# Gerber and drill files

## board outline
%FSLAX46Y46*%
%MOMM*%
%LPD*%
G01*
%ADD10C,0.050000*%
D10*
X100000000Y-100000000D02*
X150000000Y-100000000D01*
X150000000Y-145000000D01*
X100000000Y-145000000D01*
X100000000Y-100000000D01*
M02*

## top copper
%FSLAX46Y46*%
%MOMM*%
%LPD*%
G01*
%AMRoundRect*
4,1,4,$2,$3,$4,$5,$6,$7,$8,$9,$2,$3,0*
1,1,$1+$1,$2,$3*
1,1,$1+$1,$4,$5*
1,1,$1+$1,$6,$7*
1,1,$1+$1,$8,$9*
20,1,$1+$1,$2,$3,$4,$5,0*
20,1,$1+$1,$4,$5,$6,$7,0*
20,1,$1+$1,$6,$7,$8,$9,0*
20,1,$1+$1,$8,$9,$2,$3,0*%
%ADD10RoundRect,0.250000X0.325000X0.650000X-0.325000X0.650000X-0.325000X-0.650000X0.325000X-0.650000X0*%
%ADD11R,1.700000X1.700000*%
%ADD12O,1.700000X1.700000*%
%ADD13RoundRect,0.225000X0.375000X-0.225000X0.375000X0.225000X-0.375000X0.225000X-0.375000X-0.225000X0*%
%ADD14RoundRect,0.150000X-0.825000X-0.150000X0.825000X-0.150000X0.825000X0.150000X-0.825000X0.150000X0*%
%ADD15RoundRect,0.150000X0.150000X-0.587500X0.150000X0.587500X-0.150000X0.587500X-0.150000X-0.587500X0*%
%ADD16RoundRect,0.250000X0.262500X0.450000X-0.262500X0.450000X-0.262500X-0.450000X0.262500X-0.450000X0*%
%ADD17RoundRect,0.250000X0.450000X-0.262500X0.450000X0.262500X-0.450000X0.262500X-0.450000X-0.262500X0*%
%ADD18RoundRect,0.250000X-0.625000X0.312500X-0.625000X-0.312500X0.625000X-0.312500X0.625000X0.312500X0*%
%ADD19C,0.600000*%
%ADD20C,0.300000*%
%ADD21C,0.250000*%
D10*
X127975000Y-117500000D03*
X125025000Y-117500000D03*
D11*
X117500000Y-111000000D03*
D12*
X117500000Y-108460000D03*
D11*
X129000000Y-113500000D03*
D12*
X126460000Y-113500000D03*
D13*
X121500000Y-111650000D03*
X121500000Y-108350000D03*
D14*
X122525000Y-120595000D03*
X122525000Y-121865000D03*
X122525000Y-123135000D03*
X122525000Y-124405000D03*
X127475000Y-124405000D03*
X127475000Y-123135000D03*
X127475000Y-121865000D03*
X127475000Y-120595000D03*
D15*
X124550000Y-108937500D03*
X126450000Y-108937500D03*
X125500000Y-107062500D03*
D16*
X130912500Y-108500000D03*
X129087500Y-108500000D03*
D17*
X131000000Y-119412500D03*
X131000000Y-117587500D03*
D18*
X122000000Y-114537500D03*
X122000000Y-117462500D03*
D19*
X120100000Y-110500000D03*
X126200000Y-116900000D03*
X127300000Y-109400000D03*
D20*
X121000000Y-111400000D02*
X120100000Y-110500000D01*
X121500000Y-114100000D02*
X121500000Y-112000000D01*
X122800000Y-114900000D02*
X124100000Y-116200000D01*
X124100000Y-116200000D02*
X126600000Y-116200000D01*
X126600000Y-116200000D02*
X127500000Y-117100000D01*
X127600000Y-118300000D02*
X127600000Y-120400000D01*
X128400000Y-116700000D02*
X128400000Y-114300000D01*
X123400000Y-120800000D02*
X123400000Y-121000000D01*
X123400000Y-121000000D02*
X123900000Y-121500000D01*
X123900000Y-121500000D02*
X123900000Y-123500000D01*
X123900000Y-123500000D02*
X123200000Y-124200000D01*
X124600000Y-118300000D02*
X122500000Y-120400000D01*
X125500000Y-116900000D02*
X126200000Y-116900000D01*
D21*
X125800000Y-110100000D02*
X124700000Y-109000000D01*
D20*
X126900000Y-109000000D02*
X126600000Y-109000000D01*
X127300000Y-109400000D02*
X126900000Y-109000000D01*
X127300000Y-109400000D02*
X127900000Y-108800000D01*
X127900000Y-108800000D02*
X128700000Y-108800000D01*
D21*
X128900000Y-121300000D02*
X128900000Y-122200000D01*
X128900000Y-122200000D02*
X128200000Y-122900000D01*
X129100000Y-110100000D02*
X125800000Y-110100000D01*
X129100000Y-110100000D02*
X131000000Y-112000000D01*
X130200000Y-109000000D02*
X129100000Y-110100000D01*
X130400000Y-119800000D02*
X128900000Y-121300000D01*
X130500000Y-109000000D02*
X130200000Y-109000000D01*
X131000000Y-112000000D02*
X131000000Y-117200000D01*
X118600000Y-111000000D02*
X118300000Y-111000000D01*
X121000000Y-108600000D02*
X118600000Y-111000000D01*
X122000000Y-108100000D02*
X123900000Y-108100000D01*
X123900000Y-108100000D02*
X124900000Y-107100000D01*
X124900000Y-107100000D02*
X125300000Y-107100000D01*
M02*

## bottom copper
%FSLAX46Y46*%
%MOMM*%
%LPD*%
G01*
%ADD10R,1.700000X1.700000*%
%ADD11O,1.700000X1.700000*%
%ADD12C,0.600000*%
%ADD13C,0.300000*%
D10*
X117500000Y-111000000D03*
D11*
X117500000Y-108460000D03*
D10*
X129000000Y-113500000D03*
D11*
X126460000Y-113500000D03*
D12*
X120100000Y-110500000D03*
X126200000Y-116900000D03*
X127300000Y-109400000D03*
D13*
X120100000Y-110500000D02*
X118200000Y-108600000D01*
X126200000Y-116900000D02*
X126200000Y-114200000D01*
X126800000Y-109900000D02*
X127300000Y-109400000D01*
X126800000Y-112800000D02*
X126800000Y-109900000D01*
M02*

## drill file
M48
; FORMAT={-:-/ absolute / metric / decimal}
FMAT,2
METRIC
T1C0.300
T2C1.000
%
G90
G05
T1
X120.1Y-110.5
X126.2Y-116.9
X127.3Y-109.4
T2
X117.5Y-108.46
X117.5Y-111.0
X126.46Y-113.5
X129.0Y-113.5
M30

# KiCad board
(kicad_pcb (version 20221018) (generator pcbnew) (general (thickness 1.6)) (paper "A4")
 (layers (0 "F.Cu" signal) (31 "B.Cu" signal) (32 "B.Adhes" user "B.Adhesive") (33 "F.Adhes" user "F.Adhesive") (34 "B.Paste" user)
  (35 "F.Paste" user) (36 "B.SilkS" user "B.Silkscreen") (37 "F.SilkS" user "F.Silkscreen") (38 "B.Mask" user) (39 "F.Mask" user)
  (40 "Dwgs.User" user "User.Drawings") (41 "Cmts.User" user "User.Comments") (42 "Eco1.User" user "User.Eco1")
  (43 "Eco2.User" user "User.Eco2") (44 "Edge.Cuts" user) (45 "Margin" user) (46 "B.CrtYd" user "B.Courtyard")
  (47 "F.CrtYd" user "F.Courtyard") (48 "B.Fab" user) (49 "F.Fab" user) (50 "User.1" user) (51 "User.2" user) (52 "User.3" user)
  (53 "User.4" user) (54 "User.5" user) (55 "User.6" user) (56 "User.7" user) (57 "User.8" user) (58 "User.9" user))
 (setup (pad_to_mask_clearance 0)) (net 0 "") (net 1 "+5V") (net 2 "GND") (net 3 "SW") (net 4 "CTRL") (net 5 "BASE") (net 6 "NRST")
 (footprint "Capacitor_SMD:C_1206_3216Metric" (layer "F.Cu") (at 126.5 117.5 180)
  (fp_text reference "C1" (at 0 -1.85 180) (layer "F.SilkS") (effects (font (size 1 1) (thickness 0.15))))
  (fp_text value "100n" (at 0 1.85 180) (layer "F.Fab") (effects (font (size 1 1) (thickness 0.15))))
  (pad "1" smd roundrect (at -1.475 0 180) (size 1.15 1.8) (layers "F.Cu" "F.Paste" "F.Mask") (roundrect_rratio 0.217391) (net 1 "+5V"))
  (pad "2" smd roundrect (at 1.475 0 180) (size 1.15 1.8) (layers "F.Cu" "F.Paste" "F.Mask") (roundrect_rratio 0.217391) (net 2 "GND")))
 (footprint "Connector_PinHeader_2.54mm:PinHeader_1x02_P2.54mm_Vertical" (layer "F.Cu") (at 117.5 111 180)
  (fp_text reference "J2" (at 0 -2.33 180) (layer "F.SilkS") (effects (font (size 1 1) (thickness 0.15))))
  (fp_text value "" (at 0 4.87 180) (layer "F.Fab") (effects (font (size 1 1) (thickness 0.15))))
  (pad "1" thru_hole rect (at 0 0 180) (size 1.7 1.7) (drill 1) (layers "*.Cu" "*.Mask") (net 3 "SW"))
  (pad "2" thru_hole oval (at 0 2.54 180) (size 1.7 1.7) (drill 1) (layers "*.Cu" "*.Mask") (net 1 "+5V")))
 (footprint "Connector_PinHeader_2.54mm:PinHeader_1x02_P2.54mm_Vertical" (layer "F.Cu") (at 129 113.5 -90)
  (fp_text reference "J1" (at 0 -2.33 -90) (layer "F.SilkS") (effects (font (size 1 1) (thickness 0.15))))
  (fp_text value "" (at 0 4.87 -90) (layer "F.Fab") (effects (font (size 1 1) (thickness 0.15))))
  (pad "1" thru_hole rect (at 0 0 270) (size 1.7 1.7) (drill 1) (layers "*.Cu" "*.Mask") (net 1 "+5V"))
  (pad "2" thru_hole oval (at 0 2.54 270) (size 1.7 1.7) (drill 1) (layers "*.Cu" "*.Mask") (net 2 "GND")))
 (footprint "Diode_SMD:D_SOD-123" (layer "F.Cu") (at 121.5 110 90)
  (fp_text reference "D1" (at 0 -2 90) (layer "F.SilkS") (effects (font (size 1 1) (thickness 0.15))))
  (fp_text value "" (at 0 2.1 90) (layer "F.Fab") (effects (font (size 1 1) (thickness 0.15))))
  (pad "1" smd roundrect (at -1.65 0 90) (size 0.9 1.2) (layers "F.Cu" "F.Paste" "F.Mask") (roundrect_rratio 0.25) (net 1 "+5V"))
  (pad "2" smd roundrect (at 1.65 0 90) (size 0.9 1.2) (layers "F.Cu" "F.Paste" "F.Mask") (roundrect_rratio 0.25) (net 3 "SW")))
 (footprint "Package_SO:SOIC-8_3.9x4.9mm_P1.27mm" (layer "F.Cu") (at 125 122.5)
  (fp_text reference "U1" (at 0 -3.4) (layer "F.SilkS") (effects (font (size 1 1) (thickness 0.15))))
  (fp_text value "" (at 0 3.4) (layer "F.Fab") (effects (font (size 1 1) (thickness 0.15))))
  (pad "1" smd roundrect (at -2.475 -1.905) (size 1.95 0.6) (layers "F.Cu" "F.Paste" "F.Mask") (roundrect_rratio 0.25) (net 2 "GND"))
  (pad "2" smd roundrect (at -2.475 -0.635) (size 1.95 0.6) (layers "F.Cu" "F.Paste" "F.Mask") (roundrect_rratio 0.25))
  (pad "3" smd roundrect (at -2.475 0.635) (size 1.95 0.6) (layers "F.Cu" "F.Paste" "F.Mask") (roundrect_rratio 0.25))
  (pad "4" smd roundrect (at -2.475 1.905) (size 1.95 0.6) (layers "F.Cu" "F.Paste" "F.Mask") (roundrect_rratio 0.25) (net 2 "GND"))
  (pad "5" smd roundrect (at 2.475 1.905) (size 1.95 0.6) (layers "F.Cu" "F.Paste" "F.Mask") (roundrect_rratio 0.25))
  (pad "6" smd roundrect (at 2.475 0.635) (size 1.95 0.6) (layers "F.Cu" "F.Paste" "F.Mask") (roundrect_rratio 0.25) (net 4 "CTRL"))
  (pad "7" smd roundrect (at 2.475 -0.635) (size 1.95 0.6) (layers "F.Cu" "F.Paste" "F.Mask") (roundrect_rratio 0.25))
  (pad "8" smd roundrect (at 2.475 -1.905) (size 1.95 0.6) (layers "F.Cu" "F.Paste" "F.Mask") (roundrect_rratio 0.25) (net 1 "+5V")))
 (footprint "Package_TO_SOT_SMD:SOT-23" (layer "F.Cu") (at 125.5 108 90)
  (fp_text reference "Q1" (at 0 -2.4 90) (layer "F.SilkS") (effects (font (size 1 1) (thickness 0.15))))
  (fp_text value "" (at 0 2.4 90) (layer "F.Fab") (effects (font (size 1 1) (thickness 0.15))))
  (pad "1" smd roundrect (at -0.9375 -0.95 90) (size 1.475 0.6) (layers "F.Cu" "F.Paste" "F.Mask") (roundrect_rratio 0.25) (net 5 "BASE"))
  (pad "2" smd roundrect (at -0.9375 0.95 90) (size 1.475 0.6) (layers "F.Cu" "F.Paste" "F.Mask") (roundrect_rratio 0.25) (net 2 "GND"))
  (pad "3" smd roundrect (at 0.9375 0 90) (size 1.475 0.6) (layers "F.Cu" "F.Paste" "F.Mask") (roundrect_rratio 0.25) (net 3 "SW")))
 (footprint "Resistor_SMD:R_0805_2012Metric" (layer "F.Cu") (at 130 108.5 180)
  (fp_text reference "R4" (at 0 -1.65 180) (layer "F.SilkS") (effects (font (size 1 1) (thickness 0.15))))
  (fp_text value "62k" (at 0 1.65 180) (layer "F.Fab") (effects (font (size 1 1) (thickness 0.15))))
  (pad "1" smd roundrect (at -0.9125 0 180) (size 1.025 1.4) (layers "F.Cu" "F.Paste" "F.Mask") (roundrect_rratio 0.243902) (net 5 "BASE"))
  (pad "2" smd roundrect (at 0.9125 0 180) (size 1.025 1.4) (layers "F.Cu" "F.Paste" "F.Mask") (roundrect_rratio 0.243902) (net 2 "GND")))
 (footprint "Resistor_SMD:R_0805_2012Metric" (layer "F.Cu") (at 131 118.5 90)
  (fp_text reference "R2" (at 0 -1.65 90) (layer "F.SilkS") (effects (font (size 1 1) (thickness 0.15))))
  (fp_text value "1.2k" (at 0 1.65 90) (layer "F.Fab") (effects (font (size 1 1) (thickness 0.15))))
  (pad "1" smd roundrect (at -0.9125 0 90) (size 1.025 1.4) (layers "F.Cu" "F.Paste" "F.Mask") (roundrect_rratio 0.243902) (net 4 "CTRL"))
  (pad "2" smd roundrect (at 0.9125 0 90) (size 1.025 1.4) (layers "F.Cu" "F.Paste" "F.Mask") (roundrect_rratio 0.243902) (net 5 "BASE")))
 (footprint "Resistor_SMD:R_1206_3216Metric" (layer "F.Cu") (at 122 116 -90)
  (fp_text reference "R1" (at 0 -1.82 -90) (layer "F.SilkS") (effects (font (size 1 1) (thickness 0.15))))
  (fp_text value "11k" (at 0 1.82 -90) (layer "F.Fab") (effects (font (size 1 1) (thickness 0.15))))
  (pad "1" smd roundrect (at -1.4625 0 270) (size 1.125 1.75) (layers "F.Cu" "F.Paste" "F.Mask") (roundrect_rratio 0.222222) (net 1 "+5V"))
  (pad "2" smd roundrect (at 1.4625 0 270) (size 1.125 1.75) (layers "F.Cu" "F.Paste" "F.Mask") (roundrect_rratio 0.222222) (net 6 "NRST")))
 (gr_rect (start 100 100) (end 150 145) (stroke (width 0.05) (type default)) (fill none) (layer "Edge.Cuts"))
 (segment (start 121 111.4) (end 120.1 110.5) (width 0.3) (layer "F.Cu") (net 1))
 (segment (start 121.5 114.1) (end 121.5 112) (width 0.3) (layer "F.Cu") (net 1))
 (segment (start 122.8 114.9) (end 124.1 116.2) (width 0.3) (layer "F.Cu") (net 1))
 (segment (start 124.1 116.2) (end 126.6 116.2) (width 0.3) (layer "F.Cu") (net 1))
 (segment (start 126.6 116.2) (end 127.5 117.1) (width 0.3) (layer "F.Cu") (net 1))
 (segment (start 127.6 118.3) (end 127.6 120.4) (width 0.3) (layer "F.Cu") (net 1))
 (segment (start 128.4 116.7) (end 128.4 114.3) (width 0.3) (layer "F.Cu") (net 1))
 (via (at 120.1 110.5) (size 0.6) (drill 0.3) (layers "F.Cu" "B.Cu") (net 1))
 (segment (start 120.1 110.5) (end 118.2 108.6) (width 0.3) (layer "B.Cu") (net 1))
 (segment (start 123.4 120.8) (end 123.4 121) (width 0.3) (layer "F.Cu") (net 2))
 (segment (start 123.4 121) (end 123.9 121.5) (width 0.3) (layer "F.Cu") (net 2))
 (segment (start 123.9 121.5) (end 123.9 123.5) (width 0.3) (layer "F.Cu") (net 2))
 (segment (start 123.9 123.5) (end 123.2 124.2) (width 0.3) (layer "F.Cu") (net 2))
 (segment (start 124.6 118.3) (end 122.5 120.4) (width 0.3) (layer "F.Cu") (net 2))
 (segment (start 125.5 116.9) (end 126.2 116.9) (width 0.3) (layer "F.Cu") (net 2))
 (segment (start 125.8 110.1) (end 124.7 109) (width 0.25) (layer "F.Cu") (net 5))
 (segment (start 126.9 109) (end 126.6 109) (width 0.3) (layer "F.Cu") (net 2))
 (segment (start 127.3 109.4) (end 126.9 109) (width 0.3) (layer "F.Cu") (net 2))
 (segment (start 127.3 109.4) (end 127.9 108.8) (width 0.3) (layer "F.Cu") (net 2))
 (segment (start 127.9 108.8) (end 128.7 108.8) (width 0.3) (layer "F.Cu") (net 2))
 (segment (start 128.9 121.3) (end 128.9 122.2) (width 0.25) (layer "F.Cu") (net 4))
 (segment (start 128.9 122.2) (end 128.2 122.9) (width 0.25) (layer "F.Cu") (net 4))
 (segment (start 129.1 110.1) (end 125.8 110.1) (width 0.25) (layer "F.Cu") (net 5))
 (segment (start 129.1 110.1) (end 131 112) (width 0.25) (layer "F.Cu") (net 5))
 (segment (start 130.2 109) (end 129.1 110.1) (width 0.25) (layer "F.Cu") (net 5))
 (segment (start 130.4 119.8) (end 128.9 121.3) (width 0.25) (layer "F.Cu") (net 4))
 (segment (start 130.5 109) (end 130.2 109) (width 0.25) (layer "F.Cu") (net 5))
 (segment (start 131 112) (end 131 117.2) (width 0.25) (layer "F.Cu") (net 5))
 (via (at 126.2 116.9) (size 0.6) (drill 0.3) (layers "F.Cu" "B.Cu") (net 2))
 (via (at 127.3 109.4) (size 0.6) (drill 0.3) (layers "F.Cu" "B.Cu") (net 2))
 (segment (start 118.6 111) (end 118.3 111) (width 0.25) (layer "F.Cu") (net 3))
 (segment (start 121 108.6) (end 118.6 111) (width 0.25) (layer "F.Cu") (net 3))
 (segment (start 122 108.1) (end 123.9 108.1) (width 0.25) (layer "F.Cu") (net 3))
 (segment (start 123.9 108.1) (end 124.9 107.1) (width 0.25) (layer "F.Cu") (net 3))
 (segment (start 124.9 107.1) (end 125.3 107.1) (width 0.25) (layer "F.Cu") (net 3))
 (segment (start 126.2 116.9) (end 126.2 114.2) (width 0.3) (layer "B.Cu") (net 2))
 (segment (start 126.8 109.9) (end 127.3 109.4) (width 0.3) (layer "B.Cu") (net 2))
 (segment (start 126.8 112.8) (end 126.8 109.9) (width 0.3) (layer "B.Cu") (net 2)))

